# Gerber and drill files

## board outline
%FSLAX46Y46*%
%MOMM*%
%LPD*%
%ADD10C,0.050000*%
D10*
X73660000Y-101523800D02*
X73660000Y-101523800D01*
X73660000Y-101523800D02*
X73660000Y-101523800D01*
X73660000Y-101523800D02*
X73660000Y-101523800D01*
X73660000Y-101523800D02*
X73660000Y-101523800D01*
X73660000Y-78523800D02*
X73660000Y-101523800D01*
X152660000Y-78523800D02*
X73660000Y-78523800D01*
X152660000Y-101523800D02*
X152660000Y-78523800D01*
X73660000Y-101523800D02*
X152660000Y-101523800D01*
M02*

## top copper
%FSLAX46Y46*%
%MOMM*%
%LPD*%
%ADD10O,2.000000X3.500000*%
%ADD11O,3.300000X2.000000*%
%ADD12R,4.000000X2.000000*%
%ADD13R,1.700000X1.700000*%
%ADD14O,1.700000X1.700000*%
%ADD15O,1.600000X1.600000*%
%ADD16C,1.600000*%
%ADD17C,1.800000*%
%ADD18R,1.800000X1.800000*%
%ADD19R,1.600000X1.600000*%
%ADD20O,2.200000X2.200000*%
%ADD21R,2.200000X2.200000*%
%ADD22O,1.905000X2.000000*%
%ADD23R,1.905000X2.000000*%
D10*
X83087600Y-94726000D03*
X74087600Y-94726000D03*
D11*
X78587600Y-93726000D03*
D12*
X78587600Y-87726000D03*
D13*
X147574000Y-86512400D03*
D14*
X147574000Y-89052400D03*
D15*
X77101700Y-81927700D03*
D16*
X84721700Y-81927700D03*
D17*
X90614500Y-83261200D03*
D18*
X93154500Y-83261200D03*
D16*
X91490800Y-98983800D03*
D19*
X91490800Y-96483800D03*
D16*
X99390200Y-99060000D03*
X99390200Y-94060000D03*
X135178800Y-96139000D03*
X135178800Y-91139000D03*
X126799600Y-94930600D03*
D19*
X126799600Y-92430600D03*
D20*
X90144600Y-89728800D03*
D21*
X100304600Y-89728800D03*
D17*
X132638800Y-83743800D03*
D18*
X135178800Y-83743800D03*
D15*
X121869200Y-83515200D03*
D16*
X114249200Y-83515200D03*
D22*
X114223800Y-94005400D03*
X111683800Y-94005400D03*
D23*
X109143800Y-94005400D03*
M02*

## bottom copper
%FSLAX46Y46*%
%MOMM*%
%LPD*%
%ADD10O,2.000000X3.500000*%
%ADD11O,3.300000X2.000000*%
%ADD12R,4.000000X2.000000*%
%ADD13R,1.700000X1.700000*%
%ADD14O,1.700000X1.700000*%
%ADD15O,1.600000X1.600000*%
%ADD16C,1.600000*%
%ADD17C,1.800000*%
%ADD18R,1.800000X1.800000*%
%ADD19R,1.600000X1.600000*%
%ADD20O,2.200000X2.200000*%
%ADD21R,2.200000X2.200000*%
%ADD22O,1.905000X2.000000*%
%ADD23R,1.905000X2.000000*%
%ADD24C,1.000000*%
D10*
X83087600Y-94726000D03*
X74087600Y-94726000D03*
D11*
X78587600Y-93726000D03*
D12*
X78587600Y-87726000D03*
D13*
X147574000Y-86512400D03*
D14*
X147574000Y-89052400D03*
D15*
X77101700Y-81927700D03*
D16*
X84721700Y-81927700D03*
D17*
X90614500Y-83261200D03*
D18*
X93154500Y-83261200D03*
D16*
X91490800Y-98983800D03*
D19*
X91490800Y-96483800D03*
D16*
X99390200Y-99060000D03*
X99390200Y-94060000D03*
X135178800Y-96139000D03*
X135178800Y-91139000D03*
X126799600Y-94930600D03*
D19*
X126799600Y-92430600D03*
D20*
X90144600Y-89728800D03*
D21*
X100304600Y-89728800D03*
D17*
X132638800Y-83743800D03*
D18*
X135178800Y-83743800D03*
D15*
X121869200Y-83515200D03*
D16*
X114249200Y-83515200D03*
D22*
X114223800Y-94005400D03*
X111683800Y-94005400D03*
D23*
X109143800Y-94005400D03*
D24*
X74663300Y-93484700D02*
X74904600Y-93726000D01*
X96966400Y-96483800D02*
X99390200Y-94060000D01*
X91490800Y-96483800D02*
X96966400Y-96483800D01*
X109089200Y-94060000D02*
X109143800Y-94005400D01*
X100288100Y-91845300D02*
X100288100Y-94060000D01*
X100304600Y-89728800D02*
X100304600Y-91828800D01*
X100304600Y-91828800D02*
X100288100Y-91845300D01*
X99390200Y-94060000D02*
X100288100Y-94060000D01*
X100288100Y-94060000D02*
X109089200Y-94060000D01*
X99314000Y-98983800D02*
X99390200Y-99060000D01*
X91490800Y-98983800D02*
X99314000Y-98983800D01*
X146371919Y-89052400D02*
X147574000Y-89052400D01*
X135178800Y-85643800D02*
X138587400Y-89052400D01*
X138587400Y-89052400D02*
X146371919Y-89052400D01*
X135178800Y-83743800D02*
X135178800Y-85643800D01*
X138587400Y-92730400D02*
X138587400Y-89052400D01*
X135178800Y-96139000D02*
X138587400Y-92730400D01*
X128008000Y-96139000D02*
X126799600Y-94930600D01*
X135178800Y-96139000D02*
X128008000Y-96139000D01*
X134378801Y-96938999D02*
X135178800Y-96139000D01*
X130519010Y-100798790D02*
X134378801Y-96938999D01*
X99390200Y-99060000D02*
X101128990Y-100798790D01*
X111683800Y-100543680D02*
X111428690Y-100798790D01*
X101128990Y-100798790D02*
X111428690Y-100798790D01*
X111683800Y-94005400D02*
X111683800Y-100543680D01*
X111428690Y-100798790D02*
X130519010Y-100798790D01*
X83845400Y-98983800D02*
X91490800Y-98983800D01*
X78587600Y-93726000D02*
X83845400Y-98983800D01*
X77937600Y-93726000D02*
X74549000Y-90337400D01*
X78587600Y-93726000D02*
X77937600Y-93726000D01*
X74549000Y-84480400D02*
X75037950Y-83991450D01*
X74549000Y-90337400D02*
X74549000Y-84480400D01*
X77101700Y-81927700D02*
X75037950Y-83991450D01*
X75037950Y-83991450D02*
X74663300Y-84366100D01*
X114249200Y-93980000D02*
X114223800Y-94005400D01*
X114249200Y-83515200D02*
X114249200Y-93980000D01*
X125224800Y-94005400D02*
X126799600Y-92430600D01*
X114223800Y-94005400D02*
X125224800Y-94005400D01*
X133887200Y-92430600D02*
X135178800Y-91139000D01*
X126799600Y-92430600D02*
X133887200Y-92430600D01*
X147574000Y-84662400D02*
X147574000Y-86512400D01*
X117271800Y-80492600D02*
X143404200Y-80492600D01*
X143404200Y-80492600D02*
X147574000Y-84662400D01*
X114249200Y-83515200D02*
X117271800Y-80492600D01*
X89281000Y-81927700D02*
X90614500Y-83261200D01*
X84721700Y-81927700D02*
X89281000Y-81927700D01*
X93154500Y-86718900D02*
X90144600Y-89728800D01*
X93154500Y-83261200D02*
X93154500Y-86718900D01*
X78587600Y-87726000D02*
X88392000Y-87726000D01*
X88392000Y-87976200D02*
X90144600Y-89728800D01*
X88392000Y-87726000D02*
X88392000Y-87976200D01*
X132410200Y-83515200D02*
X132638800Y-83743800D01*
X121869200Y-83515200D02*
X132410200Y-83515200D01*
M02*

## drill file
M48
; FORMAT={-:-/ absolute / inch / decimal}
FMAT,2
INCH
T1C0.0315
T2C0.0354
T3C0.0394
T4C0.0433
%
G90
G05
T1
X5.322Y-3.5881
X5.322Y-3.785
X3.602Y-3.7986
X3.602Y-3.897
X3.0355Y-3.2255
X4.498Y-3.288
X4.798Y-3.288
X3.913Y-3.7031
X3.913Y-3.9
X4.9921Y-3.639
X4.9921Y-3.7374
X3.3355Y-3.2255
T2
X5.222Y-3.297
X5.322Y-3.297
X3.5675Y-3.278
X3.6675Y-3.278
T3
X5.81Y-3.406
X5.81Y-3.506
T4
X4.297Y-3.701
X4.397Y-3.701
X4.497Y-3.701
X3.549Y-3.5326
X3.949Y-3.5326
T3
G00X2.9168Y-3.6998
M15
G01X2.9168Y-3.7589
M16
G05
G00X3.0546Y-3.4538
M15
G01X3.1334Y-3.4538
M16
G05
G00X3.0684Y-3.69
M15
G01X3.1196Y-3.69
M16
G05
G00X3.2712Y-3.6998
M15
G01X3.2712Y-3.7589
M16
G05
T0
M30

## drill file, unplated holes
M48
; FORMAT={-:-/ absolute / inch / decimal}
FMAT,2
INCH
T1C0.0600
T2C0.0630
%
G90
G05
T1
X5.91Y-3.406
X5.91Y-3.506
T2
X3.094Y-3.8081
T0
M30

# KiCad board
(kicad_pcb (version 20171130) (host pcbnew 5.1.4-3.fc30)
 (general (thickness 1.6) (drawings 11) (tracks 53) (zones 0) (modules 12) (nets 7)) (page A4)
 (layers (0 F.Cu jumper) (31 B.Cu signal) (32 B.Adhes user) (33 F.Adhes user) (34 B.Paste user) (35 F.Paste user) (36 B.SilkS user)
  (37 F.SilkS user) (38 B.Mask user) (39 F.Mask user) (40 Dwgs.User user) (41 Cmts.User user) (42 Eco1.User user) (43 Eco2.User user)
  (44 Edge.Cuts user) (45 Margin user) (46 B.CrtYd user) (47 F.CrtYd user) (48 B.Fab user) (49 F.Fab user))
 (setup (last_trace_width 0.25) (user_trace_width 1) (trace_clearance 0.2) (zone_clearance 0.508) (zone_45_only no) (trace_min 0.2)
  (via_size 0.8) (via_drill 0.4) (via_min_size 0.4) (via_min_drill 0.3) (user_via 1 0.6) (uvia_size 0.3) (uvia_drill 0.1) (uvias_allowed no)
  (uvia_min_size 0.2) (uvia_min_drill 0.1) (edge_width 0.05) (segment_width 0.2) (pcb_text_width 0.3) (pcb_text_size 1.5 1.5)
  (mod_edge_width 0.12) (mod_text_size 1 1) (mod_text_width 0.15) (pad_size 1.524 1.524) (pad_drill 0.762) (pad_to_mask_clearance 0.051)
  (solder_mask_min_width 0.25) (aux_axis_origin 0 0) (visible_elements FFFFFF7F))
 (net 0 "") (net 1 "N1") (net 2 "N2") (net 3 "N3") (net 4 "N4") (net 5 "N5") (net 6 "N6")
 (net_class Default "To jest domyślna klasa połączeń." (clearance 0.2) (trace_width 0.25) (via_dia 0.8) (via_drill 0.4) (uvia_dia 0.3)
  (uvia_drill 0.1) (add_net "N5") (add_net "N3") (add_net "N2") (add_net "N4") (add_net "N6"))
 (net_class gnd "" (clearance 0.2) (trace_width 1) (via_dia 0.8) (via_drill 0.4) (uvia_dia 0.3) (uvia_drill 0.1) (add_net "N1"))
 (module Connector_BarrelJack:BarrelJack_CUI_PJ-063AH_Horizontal (layer F.Cu) (at 78.5876 87.726)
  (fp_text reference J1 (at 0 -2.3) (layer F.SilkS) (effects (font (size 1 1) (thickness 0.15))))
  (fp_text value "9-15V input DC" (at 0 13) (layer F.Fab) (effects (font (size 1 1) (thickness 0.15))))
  (pad "" np_thru_hole circle (at 0 9) (size 1.6 1.6) (drill 1.6) (layers *.Cu *.Mask))
  (pad MP thru_hole oval (at 4.5 7) (size 2 3.5) (drill oval 1 2.5) (layers *.Cu *.Mask))
  (pad MP thru_hole oval (at -4.5 7) (size 2 3.5) (drill oval 1 2.5) (layers *.Cu *.Mask))
  (pad 2 thru_hole oval (at 0 6) (size 3.3 2) (drill oval 2.3 1) (layers *.Cu *.Mask) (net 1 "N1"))
  (pad 1 thru_hole rect (at 0 0) (size 4 2) (drill oval 3 1) (layers *.Cu *.Mask) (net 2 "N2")))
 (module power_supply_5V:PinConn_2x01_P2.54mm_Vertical (layer F.Cu) (at 147.574 86.5124 270)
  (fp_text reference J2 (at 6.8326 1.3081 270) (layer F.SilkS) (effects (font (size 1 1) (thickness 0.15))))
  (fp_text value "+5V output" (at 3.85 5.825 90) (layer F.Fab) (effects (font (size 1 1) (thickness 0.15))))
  (pad 1 thru_hole rect (at 0 0 270) (size 1.7 1.7) (drill 1) (layers *.Cu *.Mask) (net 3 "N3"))
  (pad 2 thru_hole oval (at 2.54 0 270) (size 1.7 1.7) (drill 1) (layers *.Cu *.Mask) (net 1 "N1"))
  (pad "" np_thru_hole circle (at 0 -2.54 270) (size 1.524 1.524) (drill 1.524) (layers *.Cu *.Mask))
  (pad "" np_thru_hole circle (at 2.54 -2.54 270) (size 1.524 1.524) (drill 1.524) (layers *.Cu *.Mask)))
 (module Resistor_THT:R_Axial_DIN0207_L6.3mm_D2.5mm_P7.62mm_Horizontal (layer F.Cu) (at 84.7217 81.9277 180)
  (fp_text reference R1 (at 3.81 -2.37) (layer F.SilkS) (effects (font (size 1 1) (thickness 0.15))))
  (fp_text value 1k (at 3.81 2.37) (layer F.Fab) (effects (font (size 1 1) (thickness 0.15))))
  (pad 2 thru_hole oval (at 7.62 0 180) (size 1.6 1.6) (drill 0.8) (layers *.Cu *.Mask) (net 1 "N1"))
  (pad 1 thru_hole circle (at 0 0 180) (size 1.6 1.6) (drill 0.8) (layers *.Cu *.Mask) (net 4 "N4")))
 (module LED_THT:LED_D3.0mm (layer F.Cu) (at 93.1545 83.2612 180)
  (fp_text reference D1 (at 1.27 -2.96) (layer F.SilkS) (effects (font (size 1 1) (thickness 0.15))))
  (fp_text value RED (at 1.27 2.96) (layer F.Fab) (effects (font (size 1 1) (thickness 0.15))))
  (pad 2 thru_hole circle (at 2.54 0 180) (size 1.8 1.8) (drill 0.9) (layers *.Cu *.Mask) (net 4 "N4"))
  (pad 1 thru_hole rect (at 0 0 180) (size 1.8 1.8) (drill 0.9) (layers *.Cu *.Mask) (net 2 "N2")))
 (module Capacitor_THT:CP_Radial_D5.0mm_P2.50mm (layer F.Cu) (at 91.4908 96.4838 270)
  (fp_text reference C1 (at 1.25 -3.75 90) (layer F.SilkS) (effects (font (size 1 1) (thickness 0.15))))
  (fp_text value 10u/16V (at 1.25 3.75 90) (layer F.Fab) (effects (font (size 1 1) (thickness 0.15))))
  (pad 2 thru_hole circle (at 2.5 0 270) (size 1.6 1.6) (drill 0.8) (layers *.Cu *.Mask) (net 1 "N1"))
  (pad 1 thru_hole rect (at 0 0 270) (size 1.6 1.6) (drill 0.8) (layers *.Cu *.Mask) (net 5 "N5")))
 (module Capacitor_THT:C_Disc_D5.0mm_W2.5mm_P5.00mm (layer F.Cu) (at 99.3902 94.06 270)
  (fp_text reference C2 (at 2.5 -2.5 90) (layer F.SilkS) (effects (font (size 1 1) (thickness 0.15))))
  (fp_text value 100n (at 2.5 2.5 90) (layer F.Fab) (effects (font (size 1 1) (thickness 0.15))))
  (pad 2 thru_hole circle (at 5 0 270) (size 1.6 1.6) (drill 0.8) (layers *.Cu *.Mask) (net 1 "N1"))
  (pad 1 thru_hole circle (at 0 0 270) (size 1.6 1.6) (drill 0.8) (layers *.Cu *.Mask) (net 5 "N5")))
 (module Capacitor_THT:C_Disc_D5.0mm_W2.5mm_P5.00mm (layer F.Cu) (at 135.1788 91.139 270)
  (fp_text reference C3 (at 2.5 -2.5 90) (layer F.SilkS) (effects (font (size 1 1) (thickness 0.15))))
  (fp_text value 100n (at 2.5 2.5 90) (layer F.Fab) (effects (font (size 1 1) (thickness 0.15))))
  (pad 2 thru_hole circle (at 5 0 270) (size 1.6 1.6) (drill 0.8) (layers *.Cu *.Mask) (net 1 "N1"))
  (pad 1 thru_hole circle (at 0 0 270) (size 1.6 1.6) (drill 0.8) (layers *.Cu *.Mask) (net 3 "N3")))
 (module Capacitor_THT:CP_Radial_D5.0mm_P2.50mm (layer F.Cu) (at 126.7996 92.4306 270)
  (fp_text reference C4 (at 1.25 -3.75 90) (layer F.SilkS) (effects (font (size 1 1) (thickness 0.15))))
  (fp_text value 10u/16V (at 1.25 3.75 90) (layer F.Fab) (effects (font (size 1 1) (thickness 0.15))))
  (pad 2 thru_hole circle (at 2.5 0 270) (size 1.6 1.6) (drill 0.8) (layers *.Cu *.Mask) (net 1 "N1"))
  (pad 1 thru_hole rect (at 0 0 270) (size 1.6 1.6) (drill 0.8) (layers *.Cu *.Mask) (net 3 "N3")))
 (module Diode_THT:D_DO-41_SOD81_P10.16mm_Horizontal (layer F.Cu) (at 100.3046 89.7288 180)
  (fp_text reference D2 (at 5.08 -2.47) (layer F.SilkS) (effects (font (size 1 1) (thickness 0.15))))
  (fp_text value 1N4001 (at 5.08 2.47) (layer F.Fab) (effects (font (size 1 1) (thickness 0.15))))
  (pad 2 thru_hole oval (at 10.16 0 180) (size 2.2 2.2) (drill 1.1) (layers *.Cu *.Mask) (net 2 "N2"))
  (pad 1 thru_hole rect (at 0 0 180) (size 2.2 2.2) (drill 1.1) (layers *.Cu *.Mask) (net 5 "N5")))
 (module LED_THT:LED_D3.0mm (layer F.Cu) (at 135.1788 83.7438 180)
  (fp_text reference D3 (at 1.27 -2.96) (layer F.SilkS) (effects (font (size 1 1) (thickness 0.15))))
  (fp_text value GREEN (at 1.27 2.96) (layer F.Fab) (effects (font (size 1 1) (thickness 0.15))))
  (pad 2 thru_hole circle (at 2.54 0 180) (size 1.8 1.8) (drill 0.9) (layers *.Cu *.Mask) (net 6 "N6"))
  (pad 1 thru_hole rect (at 0 0 180) (size 1.8 1.8) (drill 0.9) (layers *.Cu *.Mask) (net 1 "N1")))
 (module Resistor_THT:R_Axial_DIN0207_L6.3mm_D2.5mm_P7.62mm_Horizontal (layer F.Cu) (at 114.2492 83.5152)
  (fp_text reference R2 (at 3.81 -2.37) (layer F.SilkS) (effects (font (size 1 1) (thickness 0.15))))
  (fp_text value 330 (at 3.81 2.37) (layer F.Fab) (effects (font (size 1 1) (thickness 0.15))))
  (pad 2 thru_hole oval (at 7.62 0) (size 1.6 1.6) (drill 0.8) (layers *.Cu *.Mask) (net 6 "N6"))
  (pad 1 thru_hole circle (at 0 0) (size 1.6 1.6) (drill 0.8) (layers *.Cu *.Mask) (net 3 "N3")))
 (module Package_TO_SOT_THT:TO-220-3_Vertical (layer F.Cu) (at 109.1438 94.0054)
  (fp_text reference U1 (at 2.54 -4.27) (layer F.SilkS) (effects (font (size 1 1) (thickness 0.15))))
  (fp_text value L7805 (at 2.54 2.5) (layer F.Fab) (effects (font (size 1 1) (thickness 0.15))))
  (pad 3 thru_hole oval (at 5.08 0) (size 1.905 2) (drill 1.1) (layers *.Cu *.Mask) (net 3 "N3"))
  (pad 2 thru_hole oval (at 2.54 0) (size 1.905 2) (drill 1.1) (layers *.Cu *.Mask) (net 1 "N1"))
  (pad 1 thru_hole rect (at 0 0) (size 1.905 2) (drill 1.1) (layers *.Cu *.Mask) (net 5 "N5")))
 (gr_line (start 73.66 101.5238) (end 73.66 101.5238) (layer Edge.Cuts) (width 0.05))
 (gr_line (start 73.66 101.5238) (end 73.66 101.5238) (layer Edge.Cuts) (width 0.05))
 (gr_line (start 73.66 101.5238) (end 73.66 101.5238) (layer Edge.Cuts) (width 0.05))
 (gr_line (start 73.66 101.5238) (end 73.66 101.5238) (layer Edge.Cuts) (width 0.05))
 (gr_line (start 73.66 78.5238) (end 73.66 101.5238) (layer Edge.Cuts) (width 0.05))
 (gr_line (start 152.66 78.5238) (end 73.66 78.5238) (layer Edge.Cuts) (width 0.05))
 (gr_line (start 152.66 101.5238) (end 152.66 78.5238) (layer Edge.Cuts) (width 0.05))
 (gr_line (start 73.66 101.5238) (end 152.66 101.5238) (layer Edge.Cuts) (width 0.05))
 (segment (start 74.6633 93.4847) (end 74.9046 93.726) (width 1) (layer B.Cu) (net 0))
 (segment (start 96.9664 96.4838) (end 99.3902 94.06) (width 1) (layer B.Cu) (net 5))
 (segment (start 91.4908 96.4838) (end 96.9664 96.4838) (width 1) (layer B.Cu) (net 5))
 (segment (start 109.0892 94.06) (end 109.1438 94.0054) (width 1) (layer B.Cu) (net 5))
 (segment (start 100.2881 91.8453) (end 100.2881 94.06) (width 1) (layer B.Cu) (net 5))
 (segment (start 100.3046 89.7288) (end 100.3046 91.8288) (width 1) (layer B.Cu) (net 5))
 (segment (start 100.3046 91.8288) (end 100.2881 91.8453) (width 1) (layer B.Cu) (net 5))
 (segment (start 99.3902 94.06) (end 100.2881 94.06) (width 1) (layer B.Cu) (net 5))
 (segment (start 100.2881 94.06) (end 109.0892 94.06) (width 1) (layer B.Cu) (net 5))
 (segment (start 99.314 98.9838) (end 99.3902 99.06) (width 1) (layer B.Cu) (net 1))
 (segment (start 91.4908 98.9838) (end 99.314 98.9838) (width 1) (layer B.Cu) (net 1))
 (segment (start 146.371919 89.0524) (end 147.574 89.0524) (width 1) (layer B.Cu) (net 1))
 (segment (start 135.1788 85.6438) (end 138.5874 89.0524) (width 1) (layer B.Cu) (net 1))
 (segment (start 138.5874 89.0524) (end 146.371919 89.0524) (width 1) (layer B.Cu) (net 1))
 (segment (start 135.1788 83.7438) (end 135.1788 85.6438) (width 1) (layer B.Cu) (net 1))
 (segment (start 138.5874 92.7304) (end 138.5874 89.0524) (width 1) (layer B.Cu) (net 1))
 (segment (start 135.1788 96.139) (end 138.5874 92.7304) (width 1) (layer B.Cu) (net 1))
 (segment (start 128.008 96.139) (end 126.7996 94.9306) (width 1) (layer B.Cu) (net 1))
 (segment (start 135.1788 96.139) (end 128.008 96.139) (width 1) (layer B.Cu) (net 1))
 (segment (start 134.378801 96.938999) (end 135.1788 96.139) (width 1) (layer B.Cu) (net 1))
 (segment (start 130.51901 100.79879) (end 134.378801 96.938999) (width 1) (layer B.Cu) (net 1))
 (segment (start 99.3902 99.06) (end 101.12899 100.79879) (width 1) (layer B.Cu) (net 1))
 (segment (start 111.6838 100.54368) (end 111.42869 100.79879) (width 1) (layer B.Cu) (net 1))
 (segment (start 101.12899 100.79879) (end 111.42869 100.79879) (width 1) (layer B.Cu) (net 1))
 (segment (start 111.6838 94.0054) (end 111.6838 100.54368) (width 1) (layer B.Cu) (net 1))
 (segment (start 111.42869 100.79879) (end 130.51901 100.79879) (width 1) (layer B.Cu) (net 1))
 (segment (start 83.8454 98.9838) (end 91.4908 98.9838) (width 1) (layer B.Cu) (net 1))
 (segment (start 78.5876 93.726) (end 83.8454 98.9838) (width 1) (layer B.Cu) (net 1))
 (segment (start 77.9376 93.726) (end 74.549 90.3374) (width 1) (layer B.Cu) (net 1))
 (segment (start 78.5876 93.726) (end 77.9376 93.726) (width 1) (layer B.Cu) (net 1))
 (segment (start 74.549 84.4804) (end 75.03795 83.99145) (width 1) (layer B.Cu) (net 1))
 (segment (start 74.549 90.3374) (end 74.549 84.4804) (width 1) (layer B.Cu) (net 1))
 (segment (start 77.1017 81.9277) (end 75.03795 83.99145) (width 1) (layer B.Cu) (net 1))
 (segment (start 75.03795 83.99145) (end 74.6633 84.3661) (width 1) (layer B.Cu) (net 1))
 (segment (start 114.2492 93.98) (end 114.2238 94.0054) (width 1) (layer B.Cu) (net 3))
 (segment (start 114.2492 83.5152) (end 114.2492 93.98) (width 1) (layer B.Cu) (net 3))
 (segment (start 125.2248 94.0054) (end 126.7996 92.4306) (width 1) (layer B.Cu) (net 3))
 (segment (start 114.2238 94.0054) (end 125.2248 94.0054) (width 1) (layer B.Cu) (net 3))
 (segment (start 133.8872 92.4306) (end 135.1788 91.139) (width 1) (layer B.Cu) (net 3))
 (segment (start 126.7996 92.4306) (end 133.8872 92.4306) (width 1) (layer B.Cu) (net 3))
 (segment (start 147.574 84.6624) (end 147.574 86.5124) (width 1) (layer B.Cu) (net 3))
 (segment (start 117.2718 80.4926) (end 143.4042 80.4926) (width 1) (layer B.Cu) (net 3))
 (segment (start 143.4042 80.4926) (end 147.574 84.6624) (width 1) (layer B.Cu) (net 3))
 (segment (start 114.2492 83.5152) (end 117.2718 80.4926) (width 1) (layer B.Cu) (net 3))
 (segment (start 89.281 81.9277) (end 90.6145 83.2612) (width 1) (layer B.Cu) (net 4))
 (segment (start 84.7217 81.9277) (end 89.281 81.9277) (width 1) (layer B.Cu) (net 4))
 (segment (start 93.1545 86.7189) (end 90.1446 89.7288) (width 1) (layer B.Cu) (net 2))
 (segment (start 93.1545 83.2612) (end 93.1545 86.7189) (width 1) (layer B.Cu) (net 2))
 (segment (start 78.5876 87.726) (end 88.392 87.726) (width 1) (layer B.Cu) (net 2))
 (segment (start 88.392 87.9762) (end 90.1446 89.7288) (width 1) (layer B.Cu) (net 2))
 (segment (start 88.392 87.726) (end 88.392 87.9762) (width 1) (layer B.Cu) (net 2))
 (segment (start 132.4102 83.5152) (end 132.6388 83.7438) (width 1) (layer B.Cu) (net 6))
 (segment (start 121.8692 83.5152) (end 132.4102 83.5152) (width 1) (layer B.Cu) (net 6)))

